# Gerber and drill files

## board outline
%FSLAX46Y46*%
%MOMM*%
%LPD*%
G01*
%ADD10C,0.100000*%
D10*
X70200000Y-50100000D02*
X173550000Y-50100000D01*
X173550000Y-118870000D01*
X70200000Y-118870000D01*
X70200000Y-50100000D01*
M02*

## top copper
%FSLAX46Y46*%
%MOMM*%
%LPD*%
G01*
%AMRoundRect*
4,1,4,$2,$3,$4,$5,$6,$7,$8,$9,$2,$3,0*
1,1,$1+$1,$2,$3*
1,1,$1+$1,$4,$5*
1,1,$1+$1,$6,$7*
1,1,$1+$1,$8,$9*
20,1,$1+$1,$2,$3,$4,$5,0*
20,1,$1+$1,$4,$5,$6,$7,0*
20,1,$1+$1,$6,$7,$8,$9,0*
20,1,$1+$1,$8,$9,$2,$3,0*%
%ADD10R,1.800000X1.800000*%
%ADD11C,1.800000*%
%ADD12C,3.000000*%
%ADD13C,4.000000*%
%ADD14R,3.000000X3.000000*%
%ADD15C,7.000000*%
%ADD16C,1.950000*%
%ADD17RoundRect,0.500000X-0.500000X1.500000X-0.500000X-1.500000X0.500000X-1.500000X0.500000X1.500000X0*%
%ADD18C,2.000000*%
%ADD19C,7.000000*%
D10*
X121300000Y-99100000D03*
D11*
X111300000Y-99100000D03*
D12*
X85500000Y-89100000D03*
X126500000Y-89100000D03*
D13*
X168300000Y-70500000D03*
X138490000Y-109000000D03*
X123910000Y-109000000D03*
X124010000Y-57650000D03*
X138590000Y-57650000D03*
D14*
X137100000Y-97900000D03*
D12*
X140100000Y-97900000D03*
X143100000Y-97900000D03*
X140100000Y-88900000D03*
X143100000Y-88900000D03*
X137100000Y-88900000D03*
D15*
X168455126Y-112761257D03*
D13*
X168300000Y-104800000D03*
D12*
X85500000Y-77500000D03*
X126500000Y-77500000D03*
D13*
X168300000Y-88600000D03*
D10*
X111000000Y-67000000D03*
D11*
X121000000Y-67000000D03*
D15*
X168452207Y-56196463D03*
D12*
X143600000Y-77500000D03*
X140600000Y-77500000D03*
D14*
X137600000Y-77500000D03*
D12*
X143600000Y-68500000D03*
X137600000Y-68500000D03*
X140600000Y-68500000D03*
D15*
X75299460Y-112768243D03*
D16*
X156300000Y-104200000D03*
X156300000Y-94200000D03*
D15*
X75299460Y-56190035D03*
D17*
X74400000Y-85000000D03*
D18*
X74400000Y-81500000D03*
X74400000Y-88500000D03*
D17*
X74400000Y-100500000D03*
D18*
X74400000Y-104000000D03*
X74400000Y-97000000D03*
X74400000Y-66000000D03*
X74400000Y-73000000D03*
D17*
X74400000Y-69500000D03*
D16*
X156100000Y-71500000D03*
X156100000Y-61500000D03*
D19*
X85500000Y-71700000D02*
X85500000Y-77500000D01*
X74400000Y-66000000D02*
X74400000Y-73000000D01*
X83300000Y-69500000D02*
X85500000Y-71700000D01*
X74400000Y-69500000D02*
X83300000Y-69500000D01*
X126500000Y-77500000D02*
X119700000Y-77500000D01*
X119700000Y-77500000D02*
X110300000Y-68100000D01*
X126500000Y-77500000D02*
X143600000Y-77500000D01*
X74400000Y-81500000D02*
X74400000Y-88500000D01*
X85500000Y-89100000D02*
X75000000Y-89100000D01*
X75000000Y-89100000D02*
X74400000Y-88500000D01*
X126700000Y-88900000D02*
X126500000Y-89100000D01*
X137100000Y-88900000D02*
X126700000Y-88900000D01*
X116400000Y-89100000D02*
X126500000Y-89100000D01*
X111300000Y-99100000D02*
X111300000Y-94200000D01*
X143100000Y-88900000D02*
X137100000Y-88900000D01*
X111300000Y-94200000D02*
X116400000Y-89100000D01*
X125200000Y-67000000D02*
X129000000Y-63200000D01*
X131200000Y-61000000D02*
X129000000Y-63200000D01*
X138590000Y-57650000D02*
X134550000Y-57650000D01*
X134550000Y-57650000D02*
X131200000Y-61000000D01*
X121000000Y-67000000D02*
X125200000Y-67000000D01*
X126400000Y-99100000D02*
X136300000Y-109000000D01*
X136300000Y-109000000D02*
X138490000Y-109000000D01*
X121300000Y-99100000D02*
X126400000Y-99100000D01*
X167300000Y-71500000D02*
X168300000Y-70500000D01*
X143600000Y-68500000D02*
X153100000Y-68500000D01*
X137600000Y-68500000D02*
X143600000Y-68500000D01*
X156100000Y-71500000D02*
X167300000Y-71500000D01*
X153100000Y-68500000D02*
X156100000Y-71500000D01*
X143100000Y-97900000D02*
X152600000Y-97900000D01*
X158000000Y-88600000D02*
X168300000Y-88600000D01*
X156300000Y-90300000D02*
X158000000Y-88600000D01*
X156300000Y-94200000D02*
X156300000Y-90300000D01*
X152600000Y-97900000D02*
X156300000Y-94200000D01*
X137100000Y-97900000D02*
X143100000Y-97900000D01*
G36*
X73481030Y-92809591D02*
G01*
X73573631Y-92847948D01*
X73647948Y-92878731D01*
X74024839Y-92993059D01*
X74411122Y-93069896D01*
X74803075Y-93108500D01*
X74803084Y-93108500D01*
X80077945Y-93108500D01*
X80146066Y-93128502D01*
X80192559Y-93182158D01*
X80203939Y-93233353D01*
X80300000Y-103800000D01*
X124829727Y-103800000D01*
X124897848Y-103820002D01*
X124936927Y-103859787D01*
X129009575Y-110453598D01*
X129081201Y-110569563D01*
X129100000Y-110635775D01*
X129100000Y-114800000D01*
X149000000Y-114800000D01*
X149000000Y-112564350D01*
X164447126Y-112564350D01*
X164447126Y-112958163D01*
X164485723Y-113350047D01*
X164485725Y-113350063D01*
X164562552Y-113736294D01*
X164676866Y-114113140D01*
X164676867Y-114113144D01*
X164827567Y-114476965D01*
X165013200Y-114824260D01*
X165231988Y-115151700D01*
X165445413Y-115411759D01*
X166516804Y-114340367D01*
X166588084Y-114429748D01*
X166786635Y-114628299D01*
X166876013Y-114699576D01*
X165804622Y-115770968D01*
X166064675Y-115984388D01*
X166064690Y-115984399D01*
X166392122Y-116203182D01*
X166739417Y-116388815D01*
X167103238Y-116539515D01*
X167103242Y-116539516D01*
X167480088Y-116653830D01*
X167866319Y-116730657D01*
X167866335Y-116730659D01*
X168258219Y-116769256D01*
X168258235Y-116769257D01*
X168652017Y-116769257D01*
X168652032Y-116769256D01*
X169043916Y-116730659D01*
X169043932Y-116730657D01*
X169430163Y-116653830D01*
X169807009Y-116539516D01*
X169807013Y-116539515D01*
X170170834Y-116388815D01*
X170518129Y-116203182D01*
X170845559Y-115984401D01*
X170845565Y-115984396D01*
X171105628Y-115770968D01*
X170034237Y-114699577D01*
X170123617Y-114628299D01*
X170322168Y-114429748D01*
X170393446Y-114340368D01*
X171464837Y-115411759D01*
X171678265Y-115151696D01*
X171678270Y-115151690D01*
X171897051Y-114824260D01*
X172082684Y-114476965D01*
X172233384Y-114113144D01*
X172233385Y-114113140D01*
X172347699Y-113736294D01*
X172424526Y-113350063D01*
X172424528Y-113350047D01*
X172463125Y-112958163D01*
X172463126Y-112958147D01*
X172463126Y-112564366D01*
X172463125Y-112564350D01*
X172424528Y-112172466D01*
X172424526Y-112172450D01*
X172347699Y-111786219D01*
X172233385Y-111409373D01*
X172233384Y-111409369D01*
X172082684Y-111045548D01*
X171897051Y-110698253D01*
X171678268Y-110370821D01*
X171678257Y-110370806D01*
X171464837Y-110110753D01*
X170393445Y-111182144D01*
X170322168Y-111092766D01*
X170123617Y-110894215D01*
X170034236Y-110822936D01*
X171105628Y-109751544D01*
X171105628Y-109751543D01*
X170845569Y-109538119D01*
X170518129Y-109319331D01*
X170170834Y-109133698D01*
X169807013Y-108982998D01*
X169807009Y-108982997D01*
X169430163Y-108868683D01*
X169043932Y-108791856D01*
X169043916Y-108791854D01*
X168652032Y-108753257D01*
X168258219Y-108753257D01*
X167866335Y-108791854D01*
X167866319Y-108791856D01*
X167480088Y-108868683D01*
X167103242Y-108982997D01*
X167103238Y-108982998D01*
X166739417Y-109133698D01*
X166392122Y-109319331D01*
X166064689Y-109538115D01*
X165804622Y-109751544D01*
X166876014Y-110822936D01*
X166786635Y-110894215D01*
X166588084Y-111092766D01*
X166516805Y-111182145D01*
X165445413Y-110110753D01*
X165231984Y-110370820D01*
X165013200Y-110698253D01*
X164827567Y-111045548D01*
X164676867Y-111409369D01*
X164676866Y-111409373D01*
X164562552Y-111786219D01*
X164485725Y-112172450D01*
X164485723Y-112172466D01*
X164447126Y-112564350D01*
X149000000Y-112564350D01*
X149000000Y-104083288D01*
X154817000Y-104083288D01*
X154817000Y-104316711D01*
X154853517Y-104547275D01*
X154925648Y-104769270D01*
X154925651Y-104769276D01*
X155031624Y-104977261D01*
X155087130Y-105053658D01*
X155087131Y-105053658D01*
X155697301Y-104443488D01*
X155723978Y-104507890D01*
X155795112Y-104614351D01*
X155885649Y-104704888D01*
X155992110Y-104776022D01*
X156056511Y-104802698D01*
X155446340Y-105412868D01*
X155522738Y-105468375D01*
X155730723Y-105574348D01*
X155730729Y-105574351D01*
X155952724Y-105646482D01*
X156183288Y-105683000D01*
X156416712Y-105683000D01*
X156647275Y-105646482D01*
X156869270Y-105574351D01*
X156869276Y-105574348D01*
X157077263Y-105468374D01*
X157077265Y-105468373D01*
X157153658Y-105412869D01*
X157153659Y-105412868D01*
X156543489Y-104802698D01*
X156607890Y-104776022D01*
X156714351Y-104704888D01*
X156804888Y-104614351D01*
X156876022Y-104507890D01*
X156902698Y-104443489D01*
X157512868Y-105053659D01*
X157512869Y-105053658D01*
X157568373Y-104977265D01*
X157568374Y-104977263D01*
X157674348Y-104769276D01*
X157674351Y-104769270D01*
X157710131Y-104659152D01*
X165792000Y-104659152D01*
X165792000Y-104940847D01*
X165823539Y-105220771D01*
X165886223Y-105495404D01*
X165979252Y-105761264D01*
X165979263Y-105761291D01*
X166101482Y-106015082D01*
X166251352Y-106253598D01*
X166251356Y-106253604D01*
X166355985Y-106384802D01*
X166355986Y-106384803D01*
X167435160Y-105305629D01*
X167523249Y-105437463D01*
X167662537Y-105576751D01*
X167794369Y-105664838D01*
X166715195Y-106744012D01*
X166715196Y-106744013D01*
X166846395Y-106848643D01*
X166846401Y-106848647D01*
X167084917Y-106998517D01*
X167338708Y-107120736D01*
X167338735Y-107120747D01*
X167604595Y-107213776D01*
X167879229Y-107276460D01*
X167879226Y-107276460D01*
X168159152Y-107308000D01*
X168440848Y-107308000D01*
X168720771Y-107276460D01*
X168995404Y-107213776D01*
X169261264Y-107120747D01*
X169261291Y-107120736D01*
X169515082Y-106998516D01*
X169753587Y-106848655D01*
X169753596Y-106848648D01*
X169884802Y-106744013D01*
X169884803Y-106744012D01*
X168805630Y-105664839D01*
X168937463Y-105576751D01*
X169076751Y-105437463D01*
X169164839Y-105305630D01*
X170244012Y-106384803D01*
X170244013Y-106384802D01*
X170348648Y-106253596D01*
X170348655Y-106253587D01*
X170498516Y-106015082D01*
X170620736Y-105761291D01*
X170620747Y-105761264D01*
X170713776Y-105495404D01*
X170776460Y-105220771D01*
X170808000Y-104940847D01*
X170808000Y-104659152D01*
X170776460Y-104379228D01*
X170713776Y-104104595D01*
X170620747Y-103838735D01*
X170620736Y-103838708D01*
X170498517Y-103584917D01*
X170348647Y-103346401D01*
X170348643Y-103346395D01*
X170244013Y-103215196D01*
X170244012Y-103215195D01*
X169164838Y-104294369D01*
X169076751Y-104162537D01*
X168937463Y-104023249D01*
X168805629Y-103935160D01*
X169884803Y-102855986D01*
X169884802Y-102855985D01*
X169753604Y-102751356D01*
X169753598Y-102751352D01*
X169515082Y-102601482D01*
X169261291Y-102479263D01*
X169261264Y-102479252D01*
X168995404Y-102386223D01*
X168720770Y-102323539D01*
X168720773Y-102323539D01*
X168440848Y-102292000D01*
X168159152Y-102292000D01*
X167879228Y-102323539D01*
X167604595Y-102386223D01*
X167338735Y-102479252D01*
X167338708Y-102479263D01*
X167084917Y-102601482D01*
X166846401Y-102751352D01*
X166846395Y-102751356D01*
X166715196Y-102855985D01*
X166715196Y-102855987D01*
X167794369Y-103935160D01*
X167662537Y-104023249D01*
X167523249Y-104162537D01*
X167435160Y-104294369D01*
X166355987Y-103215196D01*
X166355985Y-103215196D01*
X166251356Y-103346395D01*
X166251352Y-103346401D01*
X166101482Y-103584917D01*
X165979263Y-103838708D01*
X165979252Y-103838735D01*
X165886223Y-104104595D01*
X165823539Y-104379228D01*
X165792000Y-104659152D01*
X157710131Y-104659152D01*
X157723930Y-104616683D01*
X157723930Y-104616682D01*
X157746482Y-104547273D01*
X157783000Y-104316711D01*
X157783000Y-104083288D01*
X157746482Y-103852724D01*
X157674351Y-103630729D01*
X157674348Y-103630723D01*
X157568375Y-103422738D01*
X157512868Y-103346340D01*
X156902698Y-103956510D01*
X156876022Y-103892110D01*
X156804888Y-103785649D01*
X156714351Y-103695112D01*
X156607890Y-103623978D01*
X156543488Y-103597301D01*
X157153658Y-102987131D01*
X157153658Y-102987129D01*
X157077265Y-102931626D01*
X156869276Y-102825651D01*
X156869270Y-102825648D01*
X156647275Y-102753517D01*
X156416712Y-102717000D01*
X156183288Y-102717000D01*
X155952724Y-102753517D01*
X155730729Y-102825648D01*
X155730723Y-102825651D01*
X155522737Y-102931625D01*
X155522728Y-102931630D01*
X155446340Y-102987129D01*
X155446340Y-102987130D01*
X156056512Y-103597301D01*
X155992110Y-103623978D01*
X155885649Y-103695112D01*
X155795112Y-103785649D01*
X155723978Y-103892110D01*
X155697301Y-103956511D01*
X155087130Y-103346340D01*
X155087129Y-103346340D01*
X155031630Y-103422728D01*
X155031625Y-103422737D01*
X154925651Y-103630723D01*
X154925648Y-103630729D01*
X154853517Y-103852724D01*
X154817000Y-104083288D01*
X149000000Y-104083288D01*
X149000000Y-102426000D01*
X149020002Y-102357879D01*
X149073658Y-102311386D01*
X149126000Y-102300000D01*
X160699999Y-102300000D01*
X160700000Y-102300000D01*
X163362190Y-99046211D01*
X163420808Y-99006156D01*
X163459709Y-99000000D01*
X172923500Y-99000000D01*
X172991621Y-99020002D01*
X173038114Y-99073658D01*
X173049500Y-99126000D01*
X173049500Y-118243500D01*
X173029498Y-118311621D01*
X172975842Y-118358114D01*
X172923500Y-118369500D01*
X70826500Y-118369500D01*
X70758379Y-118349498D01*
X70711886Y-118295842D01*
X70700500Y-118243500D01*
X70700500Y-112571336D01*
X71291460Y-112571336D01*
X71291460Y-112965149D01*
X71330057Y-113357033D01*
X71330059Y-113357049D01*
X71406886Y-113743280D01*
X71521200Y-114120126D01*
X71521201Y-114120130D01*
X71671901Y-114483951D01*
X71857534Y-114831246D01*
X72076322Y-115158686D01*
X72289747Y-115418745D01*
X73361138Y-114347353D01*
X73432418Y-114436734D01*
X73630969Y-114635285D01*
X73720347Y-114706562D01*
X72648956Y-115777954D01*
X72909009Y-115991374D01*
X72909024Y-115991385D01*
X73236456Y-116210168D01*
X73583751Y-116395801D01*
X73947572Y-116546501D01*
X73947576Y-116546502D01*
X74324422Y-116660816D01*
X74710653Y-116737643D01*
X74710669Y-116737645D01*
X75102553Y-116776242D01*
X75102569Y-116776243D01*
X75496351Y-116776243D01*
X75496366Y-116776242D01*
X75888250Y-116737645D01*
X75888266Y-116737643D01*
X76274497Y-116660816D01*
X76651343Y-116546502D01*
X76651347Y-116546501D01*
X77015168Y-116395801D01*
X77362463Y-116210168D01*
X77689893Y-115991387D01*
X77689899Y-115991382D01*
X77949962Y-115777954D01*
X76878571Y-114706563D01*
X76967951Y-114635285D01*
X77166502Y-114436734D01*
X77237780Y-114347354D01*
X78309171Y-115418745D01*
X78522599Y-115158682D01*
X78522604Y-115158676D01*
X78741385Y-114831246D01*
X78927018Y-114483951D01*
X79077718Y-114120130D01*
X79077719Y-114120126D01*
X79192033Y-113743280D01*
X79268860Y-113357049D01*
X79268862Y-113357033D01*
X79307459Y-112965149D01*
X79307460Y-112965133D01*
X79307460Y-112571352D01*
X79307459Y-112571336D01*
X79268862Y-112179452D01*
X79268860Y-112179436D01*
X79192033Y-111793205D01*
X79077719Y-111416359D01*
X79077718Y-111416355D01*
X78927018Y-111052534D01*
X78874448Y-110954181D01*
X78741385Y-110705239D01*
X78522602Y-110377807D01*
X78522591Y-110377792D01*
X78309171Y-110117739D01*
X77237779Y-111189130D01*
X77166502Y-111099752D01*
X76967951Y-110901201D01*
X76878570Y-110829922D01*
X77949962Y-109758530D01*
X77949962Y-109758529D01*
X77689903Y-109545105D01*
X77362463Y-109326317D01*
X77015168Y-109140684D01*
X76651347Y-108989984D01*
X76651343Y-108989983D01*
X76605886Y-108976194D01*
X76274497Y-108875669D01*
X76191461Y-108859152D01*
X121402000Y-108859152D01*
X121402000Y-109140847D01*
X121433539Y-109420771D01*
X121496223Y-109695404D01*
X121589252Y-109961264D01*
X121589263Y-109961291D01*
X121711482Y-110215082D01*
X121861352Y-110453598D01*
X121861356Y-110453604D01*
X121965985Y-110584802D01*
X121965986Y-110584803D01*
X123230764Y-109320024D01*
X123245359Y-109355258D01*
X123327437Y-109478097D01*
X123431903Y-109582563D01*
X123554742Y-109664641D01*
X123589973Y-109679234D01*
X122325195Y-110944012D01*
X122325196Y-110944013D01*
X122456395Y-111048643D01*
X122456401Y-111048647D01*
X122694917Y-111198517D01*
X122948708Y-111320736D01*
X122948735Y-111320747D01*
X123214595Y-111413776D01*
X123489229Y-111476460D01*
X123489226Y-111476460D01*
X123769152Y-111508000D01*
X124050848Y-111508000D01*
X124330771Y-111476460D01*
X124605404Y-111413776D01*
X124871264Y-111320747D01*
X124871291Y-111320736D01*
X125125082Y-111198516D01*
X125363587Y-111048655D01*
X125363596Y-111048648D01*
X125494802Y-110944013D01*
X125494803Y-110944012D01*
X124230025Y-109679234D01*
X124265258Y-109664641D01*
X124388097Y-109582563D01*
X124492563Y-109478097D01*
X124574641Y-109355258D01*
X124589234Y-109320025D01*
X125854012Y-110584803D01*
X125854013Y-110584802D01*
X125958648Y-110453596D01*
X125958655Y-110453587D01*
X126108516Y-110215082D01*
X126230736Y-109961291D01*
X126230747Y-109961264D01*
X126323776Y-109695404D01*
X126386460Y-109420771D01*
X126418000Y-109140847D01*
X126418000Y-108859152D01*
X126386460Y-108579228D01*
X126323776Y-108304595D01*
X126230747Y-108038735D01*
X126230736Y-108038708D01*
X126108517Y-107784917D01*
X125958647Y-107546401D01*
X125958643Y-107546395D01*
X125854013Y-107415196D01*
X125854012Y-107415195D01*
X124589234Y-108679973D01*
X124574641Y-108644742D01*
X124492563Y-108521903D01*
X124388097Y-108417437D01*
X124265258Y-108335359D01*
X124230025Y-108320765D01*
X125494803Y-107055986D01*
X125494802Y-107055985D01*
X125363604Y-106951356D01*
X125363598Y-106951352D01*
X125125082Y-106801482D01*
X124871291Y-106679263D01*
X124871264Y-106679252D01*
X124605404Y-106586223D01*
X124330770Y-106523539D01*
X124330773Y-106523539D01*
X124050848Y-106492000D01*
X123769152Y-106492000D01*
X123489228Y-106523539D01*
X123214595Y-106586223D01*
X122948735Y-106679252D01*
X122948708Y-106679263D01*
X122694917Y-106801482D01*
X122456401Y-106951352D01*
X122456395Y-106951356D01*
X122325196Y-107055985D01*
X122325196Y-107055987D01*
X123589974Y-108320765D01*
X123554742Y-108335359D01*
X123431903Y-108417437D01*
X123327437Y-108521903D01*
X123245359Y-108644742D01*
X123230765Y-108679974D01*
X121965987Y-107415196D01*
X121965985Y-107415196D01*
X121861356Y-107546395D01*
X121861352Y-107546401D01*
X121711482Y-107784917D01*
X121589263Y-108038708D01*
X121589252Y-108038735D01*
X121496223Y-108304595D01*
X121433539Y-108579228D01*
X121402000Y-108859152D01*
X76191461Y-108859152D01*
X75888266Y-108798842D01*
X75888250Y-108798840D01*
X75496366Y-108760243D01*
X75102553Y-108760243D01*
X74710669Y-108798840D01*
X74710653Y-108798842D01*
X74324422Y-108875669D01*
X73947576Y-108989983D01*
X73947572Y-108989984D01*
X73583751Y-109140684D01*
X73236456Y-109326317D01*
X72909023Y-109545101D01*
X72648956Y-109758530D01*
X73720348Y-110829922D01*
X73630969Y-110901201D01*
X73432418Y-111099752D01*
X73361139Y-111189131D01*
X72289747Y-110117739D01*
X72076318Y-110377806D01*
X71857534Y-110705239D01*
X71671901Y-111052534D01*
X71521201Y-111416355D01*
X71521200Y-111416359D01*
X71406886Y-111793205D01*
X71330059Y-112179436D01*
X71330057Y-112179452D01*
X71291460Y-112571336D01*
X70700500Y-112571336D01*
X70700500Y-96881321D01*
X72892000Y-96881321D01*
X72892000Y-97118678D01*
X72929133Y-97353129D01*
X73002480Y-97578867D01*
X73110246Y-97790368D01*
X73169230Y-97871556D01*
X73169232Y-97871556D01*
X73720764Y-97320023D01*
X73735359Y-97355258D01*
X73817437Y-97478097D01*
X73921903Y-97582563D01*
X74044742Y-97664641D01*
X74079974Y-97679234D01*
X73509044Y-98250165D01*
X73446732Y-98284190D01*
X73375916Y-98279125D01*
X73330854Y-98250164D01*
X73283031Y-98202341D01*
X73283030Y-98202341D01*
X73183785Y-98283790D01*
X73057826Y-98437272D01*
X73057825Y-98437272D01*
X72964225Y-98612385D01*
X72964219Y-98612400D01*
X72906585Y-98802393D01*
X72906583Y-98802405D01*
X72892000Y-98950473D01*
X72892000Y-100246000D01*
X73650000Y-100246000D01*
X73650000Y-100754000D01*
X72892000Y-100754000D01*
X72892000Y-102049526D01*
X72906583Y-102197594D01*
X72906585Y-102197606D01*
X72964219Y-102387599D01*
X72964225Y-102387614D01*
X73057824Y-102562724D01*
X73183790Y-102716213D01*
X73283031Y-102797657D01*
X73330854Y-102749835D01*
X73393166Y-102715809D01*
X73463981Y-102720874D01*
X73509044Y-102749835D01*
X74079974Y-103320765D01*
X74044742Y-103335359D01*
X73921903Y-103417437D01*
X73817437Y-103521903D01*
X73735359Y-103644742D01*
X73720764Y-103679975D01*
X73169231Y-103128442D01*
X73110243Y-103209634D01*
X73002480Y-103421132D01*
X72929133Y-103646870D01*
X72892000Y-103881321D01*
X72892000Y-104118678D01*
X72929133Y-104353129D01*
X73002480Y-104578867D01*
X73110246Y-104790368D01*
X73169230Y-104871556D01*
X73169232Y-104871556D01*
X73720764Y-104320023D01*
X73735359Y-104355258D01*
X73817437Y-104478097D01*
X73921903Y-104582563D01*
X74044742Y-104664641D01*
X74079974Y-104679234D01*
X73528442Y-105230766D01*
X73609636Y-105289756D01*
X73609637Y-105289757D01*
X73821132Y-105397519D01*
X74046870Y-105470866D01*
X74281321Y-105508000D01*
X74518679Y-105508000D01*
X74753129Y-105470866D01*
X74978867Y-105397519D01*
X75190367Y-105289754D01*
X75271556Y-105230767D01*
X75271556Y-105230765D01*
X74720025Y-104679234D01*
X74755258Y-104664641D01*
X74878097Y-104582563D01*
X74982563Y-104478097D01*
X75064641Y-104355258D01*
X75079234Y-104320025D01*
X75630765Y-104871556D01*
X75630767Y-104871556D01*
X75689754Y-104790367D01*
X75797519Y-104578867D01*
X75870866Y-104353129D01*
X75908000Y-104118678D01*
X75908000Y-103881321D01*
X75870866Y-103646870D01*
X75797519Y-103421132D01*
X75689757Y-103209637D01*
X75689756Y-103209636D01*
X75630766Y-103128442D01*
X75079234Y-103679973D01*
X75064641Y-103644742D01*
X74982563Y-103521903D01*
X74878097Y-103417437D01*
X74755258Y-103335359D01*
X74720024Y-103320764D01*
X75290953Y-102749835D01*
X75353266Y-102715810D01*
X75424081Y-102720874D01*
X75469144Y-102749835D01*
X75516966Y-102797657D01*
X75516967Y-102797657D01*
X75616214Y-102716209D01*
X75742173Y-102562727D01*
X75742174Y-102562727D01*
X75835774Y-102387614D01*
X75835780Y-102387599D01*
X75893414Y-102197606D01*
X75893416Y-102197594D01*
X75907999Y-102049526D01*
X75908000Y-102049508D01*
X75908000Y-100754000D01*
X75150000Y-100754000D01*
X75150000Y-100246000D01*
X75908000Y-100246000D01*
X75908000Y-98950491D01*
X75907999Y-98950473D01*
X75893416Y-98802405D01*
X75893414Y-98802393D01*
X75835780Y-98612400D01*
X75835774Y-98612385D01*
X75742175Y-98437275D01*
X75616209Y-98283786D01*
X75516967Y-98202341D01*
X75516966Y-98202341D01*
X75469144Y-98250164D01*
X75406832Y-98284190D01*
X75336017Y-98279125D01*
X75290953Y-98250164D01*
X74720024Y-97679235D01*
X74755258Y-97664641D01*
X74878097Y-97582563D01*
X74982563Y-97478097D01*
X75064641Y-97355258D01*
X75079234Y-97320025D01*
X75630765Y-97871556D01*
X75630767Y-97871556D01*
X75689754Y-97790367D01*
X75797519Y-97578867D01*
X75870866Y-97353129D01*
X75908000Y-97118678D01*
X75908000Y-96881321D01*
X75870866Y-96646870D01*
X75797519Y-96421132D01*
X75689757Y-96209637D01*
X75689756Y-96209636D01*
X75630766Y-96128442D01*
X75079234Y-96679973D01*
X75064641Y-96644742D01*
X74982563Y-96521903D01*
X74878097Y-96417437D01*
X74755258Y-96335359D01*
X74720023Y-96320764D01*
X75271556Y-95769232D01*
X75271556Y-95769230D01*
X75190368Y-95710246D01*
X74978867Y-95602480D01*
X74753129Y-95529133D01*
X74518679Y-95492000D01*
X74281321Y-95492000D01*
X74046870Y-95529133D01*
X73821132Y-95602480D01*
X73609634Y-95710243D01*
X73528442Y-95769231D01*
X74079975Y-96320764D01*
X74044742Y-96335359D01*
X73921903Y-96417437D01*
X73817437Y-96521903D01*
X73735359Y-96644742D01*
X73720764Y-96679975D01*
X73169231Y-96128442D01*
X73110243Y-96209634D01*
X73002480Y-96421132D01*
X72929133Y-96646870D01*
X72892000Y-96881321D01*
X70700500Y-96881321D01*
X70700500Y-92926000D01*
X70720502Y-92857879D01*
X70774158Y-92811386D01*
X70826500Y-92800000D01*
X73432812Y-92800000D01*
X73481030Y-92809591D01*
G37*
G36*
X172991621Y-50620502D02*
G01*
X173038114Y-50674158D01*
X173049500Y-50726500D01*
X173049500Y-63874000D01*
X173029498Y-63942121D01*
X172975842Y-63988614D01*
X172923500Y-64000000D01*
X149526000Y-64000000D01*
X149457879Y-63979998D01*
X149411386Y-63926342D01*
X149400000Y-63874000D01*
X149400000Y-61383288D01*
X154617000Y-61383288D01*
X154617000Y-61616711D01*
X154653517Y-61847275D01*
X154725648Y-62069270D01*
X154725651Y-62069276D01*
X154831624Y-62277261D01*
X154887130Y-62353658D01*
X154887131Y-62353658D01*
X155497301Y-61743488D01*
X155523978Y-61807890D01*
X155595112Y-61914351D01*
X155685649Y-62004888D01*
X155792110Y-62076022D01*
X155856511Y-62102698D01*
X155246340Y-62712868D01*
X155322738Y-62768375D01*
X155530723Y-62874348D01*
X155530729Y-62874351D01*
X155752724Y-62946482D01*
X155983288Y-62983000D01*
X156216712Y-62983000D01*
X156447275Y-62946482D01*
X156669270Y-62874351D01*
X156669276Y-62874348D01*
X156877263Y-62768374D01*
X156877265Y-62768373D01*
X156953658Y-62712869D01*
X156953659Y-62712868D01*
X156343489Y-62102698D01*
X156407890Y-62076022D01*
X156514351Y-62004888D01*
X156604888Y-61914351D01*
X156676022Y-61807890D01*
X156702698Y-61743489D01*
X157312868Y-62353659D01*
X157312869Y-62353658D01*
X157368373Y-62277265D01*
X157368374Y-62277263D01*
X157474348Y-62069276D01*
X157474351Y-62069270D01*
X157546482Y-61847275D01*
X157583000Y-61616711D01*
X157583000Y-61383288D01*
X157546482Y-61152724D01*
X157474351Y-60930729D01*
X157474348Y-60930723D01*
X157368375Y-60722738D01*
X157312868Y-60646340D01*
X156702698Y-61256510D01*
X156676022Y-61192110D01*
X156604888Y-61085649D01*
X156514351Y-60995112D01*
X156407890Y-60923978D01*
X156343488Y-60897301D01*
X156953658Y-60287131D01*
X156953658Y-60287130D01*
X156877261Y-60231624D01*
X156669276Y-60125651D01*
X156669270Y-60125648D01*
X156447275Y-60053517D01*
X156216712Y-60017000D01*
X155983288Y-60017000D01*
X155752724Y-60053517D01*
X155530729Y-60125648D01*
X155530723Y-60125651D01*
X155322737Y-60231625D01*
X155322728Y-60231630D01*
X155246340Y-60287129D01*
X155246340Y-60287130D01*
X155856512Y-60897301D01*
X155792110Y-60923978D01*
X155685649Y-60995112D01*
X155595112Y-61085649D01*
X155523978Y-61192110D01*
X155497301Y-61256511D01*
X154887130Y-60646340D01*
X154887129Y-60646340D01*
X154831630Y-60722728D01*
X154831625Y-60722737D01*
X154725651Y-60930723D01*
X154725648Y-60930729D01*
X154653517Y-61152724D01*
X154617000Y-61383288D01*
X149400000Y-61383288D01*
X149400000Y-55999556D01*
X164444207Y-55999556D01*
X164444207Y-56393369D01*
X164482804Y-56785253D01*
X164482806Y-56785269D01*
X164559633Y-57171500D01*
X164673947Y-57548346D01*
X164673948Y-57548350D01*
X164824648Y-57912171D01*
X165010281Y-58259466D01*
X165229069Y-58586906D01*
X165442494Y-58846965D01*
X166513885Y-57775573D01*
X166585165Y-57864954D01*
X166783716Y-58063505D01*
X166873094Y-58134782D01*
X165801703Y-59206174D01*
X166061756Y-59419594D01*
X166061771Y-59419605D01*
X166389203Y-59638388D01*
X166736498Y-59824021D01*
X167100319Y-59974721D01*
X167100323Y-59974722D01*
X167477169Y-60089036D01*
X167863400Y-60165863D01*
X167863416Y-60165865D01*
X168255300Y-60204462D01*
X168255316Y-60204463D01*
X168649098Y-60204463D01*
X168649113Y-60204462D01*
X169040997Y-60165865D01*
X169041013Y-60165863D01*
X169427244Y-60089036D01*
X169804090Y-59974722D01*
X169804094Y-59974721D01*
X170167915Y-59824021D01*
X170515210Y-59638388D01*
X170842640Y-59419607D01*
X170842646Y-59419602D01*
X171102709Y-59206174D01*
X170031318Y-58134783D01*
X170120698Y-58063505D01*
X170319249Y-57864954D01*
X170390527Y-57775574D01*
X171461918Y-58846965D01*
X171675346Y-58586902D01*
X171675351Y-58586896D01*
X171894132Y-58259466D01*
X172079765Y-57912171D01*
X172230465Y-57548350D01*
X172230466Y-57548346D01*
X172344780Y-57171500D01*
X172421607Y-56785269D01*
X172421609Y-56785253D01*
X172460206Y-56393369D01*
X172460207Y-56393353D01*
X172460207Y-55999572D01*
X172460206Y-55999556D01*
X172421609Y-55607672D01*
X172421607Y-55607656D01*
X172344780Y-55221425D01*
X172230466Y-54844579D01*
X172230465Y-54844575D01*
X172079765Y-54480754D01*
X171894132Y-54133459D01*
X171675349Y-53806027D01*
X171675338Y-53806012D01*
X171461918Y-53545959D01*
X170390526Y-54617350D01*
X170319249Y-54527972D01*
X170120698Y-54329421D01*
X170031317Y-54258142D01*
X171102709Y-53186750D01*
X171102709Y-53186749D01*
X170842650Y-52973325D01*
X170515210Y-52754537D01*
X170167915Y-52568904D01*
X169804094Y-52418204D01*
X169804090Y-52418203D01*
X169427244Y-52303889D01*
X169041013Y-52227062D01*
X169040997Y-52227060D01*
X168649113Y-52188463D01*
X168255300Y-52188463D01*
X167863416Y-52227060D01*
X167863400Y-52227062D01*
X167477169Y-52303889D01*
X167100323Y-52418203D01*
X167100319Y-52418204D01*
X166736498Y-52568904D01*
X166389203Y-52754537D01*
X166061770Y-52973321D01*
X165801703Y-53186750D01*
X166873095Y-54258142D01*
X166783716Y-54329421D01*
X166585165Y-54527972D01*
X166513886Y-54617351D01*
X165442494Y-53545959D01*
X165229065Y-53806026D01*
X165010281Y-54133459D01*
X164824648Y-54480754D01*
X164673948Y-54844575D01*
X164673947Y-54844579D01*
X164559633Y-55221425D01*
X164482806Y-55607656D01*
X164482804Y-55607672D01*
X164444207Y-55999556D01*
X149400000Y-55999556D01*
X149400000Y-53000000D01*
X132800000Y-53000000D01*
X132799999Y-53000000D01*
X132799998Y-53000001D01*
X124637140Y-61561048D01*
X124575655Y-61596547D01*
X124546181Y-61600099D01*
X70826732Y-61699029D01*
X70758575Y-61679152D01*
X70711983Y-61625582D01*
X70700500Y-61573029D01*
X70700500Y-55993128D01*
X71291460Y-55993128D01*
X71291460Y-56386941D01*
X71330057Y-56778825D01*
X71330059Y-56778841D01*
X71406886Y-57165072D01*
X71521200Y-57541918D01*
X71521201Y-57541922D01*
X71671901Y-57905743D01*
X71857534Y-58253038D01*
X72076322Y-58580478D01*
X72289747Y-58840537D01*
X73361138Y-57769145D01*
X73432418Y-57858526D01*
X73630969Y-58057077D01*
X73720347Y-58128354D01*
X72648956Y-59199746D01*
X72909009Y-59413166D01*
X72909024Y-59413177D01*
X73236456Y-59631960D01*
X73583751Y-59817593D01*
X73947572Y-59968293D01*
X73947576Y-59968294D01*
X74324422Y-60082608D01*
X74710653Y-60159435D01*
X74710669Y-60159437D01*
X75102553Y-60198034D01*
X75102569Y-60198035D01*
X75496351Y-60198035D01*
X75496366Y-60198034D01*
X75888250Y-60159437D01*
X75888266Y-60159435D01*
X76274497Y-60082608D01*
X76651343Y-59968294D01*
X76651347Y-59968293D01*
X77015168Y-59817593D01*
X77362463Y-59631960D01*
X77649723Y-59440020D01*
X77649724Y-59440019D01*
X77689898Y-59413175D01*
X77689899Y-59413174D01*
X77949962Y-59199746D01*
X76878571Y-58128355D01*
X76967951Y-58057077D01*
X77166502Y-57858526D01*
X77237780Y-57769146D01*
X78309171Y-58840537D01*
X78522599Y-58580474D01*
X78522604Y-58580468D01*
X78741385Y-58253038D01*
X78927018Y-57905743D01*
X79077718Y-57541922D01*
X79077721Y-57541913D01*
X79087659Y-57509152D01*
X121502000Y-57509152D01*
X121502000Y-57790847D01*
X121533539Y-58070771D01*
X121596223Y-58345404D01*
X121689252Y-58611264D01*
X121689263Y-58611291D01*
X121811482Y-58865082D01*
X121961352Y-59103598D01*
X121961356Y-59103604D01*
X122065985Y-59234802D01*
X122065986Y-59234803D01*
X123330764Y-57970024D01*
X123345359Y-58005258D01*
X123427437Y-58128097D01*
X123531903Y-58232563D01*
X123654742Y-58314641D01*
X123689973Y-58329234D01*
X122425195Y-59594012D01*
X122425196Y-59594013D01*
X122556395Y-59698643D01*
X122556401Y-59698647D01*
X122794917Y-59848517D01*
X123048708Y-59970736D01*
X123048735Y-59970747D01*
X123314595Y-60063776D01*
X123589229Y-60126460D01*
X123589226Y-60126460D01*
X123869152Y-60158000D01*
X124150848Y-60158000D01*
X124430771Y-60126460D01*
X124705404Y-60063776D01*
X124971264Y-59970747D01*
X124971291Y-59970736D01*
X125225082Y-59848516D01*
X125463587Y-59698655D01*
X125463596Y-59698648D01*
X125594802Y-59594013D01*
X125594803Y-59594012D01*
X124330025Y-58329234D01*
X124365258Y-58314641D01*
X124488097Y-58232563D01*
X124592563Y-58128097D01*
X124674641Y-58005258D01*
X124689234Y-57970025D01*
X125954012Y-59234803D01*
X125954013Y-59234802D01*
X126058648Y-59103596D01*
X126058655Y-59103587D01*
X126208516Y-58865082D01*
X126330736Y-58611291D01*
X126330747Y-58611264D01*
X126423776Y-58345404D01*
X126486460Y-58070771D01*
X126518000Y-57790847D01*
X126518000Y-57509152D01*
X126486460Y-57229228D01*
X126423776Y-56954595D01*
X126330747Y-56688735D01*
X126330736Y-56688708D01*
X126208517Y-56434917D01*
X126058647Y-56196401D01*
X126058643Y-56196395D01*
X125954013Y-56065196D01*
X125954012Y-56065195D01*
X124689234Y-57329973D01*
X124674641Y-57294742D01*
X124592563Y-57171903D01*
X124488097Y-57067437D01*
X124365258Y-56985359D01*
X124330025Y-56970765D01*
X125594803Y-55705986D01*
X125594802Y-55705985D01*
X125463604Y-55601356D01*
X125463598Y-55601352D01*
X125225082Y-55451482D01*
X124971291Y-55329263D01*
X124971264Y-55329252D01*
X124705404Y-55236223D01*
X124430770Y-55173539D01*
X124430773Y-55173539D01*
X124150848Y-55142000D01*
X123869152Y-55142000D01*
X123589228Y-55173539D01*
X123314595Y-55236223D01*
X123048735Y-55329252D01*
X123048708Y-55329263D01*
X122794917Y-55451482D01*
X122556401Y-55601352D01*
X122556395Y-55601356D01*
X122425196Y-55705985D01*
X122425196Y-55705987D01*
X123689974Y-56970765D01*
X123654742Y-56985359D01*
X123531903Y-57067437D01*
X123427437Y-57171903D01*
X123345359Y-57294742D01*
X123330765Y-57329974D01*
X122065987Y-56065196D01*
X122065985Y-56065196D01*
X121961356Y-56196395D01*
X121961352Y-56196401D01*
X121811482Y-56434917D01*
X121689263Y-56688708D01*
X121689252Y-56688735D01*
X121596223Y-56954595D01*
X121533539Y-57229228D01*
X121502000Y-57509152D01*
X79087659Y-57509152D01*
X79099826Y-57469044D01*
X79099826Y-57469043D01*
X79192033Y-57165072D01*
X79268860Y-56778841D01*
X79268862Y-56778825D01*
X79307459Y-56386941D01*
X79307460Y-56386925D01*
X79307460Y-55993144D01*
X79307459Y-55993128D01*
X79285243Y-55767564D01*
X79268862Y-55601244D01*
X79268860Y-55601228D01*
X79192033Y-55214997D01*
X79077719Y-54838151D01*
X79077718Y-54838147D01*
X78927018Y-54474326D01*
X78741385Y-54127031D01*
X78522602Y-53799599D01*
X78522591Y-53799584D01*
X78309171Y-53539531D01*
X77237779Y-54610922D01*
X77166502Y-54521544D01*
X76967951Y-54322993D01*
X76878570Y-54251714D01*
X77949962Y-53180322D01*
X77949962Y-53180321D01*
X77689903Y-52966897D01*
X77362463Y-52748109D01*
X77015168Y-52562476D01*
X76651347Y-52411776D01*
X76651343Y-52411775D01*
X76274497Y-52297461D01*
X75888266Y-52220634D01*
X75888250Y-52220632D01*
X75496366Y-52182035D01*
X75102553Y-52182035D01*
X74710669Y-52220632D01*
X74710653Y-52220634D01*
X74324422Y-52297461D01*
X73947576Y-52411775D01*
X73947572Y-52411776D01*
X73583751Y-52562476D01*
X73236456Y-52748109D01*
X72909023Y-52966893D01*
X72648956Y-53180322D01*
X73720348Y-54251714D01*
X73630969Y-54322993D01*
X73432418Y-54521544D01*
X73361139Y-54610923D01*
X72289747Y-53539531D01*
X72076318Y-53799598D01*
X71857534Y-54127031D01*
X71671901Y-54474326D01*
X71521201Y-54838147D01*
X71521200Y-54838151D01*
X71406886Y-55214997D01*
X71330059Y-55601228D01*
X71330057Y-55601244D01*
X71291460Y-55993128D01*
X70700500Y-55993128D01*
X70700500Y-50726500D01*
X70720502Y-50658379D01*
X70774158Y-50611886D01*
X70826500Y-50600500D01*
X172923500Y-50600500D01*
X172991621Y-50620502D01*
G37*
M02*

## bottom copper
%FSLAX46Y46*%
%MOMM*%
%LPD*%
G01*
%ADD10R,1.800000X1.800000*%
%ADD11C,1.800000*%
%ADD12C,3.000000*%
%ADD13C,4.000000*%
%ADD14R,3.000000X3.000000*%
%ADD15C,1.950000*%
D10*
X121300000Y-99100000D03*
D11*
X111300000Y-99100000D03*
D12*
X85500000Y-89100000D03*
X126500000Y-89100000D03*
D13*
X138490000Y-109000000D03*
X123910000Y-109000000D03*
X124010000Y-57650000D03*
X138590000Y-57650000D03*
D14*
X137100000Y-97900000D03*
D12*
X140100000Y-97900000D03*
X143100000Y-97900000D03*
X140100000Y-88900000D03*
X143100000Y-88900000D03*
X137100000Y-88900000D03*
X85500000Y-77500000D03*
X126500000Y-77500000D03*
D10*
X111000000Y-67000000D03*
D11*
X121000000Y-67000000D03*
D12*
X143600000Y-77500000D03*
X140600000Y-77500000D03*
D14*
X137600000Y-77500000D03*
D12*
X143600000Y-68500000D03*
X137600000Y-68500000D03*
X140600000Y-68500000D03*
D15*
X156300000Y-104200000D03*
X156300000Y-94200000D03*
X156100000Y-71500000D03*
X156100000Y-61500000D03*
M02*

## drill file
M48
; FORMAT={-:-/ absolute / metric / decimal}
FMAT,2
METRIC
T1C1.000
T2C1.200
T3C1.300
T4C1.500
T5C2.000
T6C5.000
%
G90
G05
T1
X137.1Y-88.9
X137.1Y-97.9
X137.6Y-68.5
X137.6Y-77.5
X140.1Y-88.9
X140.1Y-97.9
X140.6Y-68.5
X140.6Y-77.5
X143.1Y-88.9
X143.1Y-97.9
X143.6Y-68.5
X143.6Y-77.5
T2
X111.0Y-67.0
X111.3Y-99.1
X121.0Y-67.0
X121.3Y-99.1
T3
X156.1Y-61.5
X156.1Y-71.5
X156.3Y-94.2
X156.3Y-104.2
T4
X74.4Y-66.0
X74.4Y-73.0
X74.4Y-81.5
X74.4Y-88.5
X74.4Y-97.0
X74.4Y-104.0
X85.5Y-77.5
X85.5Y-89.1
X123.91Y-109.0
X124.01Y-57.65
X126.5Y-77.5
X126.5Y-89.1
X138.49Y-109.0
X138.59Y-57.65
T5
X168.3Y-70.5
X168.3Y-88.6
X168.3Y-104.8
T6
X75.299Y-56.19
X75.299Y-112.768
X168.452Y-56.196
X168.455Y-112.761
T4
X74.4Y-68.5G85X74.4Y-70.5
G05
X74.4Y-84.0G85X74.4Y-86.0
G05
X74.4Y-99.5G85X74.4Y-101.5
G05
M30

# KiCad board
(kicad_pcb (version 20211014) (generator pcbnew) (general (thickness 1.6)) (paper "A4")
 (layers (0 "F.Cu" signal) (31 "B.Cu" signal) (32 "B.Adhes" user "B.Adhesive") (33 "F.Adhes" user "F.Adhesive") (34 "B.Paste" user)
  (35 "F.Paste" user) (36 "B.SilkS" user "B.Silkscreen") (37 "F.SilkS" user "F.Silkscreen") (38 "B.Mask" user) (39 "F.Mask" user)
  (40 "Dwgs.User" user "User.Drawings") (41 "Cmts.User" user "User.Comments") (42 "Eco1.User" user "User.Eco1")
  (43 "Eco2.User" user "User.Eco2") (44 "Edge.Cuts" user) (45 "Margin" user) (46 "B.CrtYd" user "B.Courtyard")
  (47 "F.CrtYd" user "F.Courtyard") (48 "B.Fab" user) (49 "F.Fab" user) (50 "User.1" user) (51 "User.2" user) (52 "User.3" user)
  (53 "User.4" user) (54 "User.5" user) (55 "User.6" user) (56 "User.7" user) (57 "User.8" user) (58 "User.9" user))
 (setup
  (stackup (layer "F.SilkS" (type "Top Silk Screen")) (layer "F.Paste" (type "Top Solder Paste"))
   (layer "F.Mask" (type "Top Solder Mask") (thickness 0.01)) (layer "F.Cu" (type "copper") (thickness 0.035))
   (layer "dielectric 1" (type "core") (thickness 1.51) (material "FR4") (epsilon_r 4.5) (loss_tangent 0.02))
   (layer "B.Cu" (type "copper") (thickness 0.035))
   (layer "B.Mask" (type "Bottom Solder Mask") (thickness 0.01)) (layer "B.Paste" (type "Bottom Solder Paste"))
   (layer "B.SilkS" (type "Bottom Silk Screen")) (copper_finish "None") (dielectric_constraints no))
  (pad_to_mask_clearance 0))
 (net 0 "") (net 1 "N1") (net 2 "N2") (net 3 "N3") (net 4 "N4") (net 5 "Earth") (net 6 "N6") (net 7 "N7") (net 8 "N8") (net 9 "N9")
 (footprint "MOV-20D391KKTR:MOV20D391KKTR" (layer "F.Cu") (at 121.3 99.1 180)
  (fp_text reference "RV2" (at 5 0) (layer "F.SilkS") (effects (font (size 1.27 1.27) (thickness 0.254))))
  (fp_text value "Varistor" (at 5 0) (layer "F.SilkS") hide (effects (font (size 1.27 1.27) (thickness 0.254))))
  (pad "1" thru_hole rect locked (at 0 0 180) (size 1.8 1.8) (drill 1.2) (layers *.Cu *.Mask) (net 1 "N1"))
  (pad "2" thru_hole circle locked (at 10 0 180) (size 1.8 1.8) (drill 1.2) (layers *.Cu *.Mask) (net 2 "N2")))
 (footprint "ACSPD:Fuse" (layer "F.Cu") (at 106 89.1)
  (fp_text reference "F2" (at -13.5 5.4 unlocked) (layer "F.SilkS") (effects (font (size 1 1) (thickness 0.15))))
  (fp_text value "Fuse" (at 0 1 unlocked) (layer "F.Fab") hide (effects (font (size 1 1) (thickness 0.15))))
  (pad "1" thru_hole circle (at -20.5 0) (size 3 3) (drill 1.5) (layers *.Cu *.Mask) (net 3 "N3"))
  (pad "2" thru_hole circle (at 20.5 0) (size 3 3) (drill 1.5) (layers *.Cu *.Mask) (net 2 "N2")))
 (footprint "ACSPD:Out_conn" (layer "F.Cu") (at 168.3 70.5)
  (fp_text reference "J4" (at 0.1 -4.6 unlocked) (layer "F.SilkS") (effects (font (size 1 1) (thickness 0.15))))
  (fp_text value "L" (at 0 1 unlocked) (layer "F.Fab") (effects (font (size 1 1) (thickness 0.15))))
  (pad "1" thru_hole circle (at 0 0) (size 4 4) (drill 2) (layers *.Cu *.Mask) (remove_unused_layers) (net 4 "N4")))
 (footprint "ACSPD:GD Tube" (layer "F.Cu") (at 131.2 109 180)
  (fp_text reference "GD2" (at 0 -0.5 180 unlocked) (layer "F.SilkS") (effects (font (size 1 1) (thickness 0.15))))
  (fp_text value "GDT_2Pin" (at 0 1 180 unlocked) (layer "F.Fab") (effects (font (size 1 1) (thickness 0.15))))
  (pad "1" thru_hole circle (at -7.29 0 180) (size 4 4) (drill 1.5) (layers *.Cu *.Mask) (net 1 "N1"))
  (pad "3" thru_hole circle (at 7.29 0 180) (size 4 4) (drill 1.5) (layers *.Cu *.Mask) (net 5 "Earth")))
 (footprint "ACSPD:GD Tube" (layer "F.Cu") (at 131.3 57.65)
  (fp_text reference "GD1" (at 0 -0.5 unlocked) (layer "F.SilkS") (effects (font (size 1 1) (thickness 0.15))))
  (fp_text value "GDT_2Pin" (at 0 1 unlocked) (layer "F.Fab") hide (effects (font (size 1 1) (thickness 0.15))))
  (pad "1" thru_hole circle (at -7.29 0) (size 4 4) (drill 1.5) (layers *.Cu *.Mask) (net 5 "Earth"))
  (pad "3" thru_hole circle (at 7.29 0) (size 4 4) (drill 1.5) (layers *.Cu *.Mask) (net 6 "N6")))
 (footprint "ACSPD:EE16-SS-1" (layer "F.Cu") (at 140.1 93.4 180)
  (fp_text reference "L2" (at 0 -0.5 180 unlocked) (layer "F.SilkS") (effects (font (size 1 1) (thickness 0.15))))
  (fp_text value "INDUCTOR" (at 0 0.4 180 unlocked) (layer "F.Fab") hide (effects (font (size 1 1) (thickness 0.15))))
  (pad "1" thru_hole rect (at 3 -4.5 180) (size 3 3) (drill 1) (layers *.Cu *.Mask) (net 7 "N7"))
  (pad "1" thru_hole circle (at 0 -4.5 180) (size 3 3) (drill 1) (layers *.Cu *.Mask) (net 7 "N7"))
  (pad "1" thru_hole circle (at -3 -4.5 180) (size 3 3) (drill 1) (layers *.Cu *.Mask) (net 7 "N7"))
  (pad "2" thru_hole circle (at 0 4.5 180) (size 3 3) (drill 1) (layers *.Cu *.Mask) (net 2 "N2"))
  (pad "2" thru_hole circle (at -3 4.5 180) (size 3 3) (drill 1) (layers *.Cu *.Mask) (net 2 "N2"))
  (pad "2" thru_hole circle (at 3 4.5 180) (size 3 3) (drill 1) (layers *.Cu *.Mask) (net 2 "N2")))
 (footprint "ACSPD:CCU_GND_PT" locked (layer "F.Cu") (at 168.455126 112.761257)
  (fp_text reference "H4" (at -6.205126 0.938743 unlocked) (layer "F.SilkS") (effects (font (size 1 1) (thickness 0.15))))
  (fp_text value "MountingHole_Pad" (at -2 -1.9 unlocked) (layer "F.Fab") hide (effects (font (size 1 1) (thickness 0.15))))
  (pad "1" thru_hole circle locked (at 0 0) (size 7 7) (drill 5) (layers *.Cu *.Mask) (remove_unused_layers) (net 5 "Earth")))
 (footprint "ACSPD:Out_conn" (layer "F.Cu") (at 168.3 104.8)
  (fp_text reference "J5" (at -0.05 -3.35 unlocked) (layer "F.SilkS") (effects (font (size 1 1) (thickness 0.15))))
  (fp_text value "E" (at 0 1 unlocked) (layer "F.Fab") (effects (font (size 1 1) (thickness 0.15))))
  (pad "1" thru_hole circle (at 0 0) (size 4 4) (drill 2) (layers *.Cu *.Mask) (remove_unused_layers) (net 5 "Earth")))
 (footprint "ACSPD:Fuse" (layer "F.Cu") (at 106 77.5)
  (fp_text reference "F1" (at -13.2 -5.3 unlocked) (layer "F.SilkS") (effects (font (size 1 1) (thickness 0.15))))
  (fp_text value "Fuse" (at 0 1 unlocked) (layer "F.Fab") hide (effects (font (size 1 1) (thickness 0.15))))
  (pad "1" thru_hole circle (at -20.5 0) (size 3 3) (drill 1.5) (layers *.Cu *.Mask) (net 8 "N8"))
  (pad "2" thru_hole circle (at 20.5 0) (size 3 3) (drill 1.5) (layers *.Cu *.Mask) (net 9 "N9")))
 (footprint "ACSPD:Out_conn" (layer "F.Cu") (at 168.3 88.6)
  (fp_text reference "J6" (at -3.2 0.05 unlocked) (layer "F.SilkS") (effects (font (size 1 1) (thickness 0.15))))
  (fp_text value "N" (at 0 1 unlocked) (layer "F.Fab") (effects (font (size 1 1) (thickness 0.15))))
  (pad "1" thru_hole circle (at 0 0) (size 4 4) (drill 2) (layers *.Cu *.Mask) (remove_unused_layers) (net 7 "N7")))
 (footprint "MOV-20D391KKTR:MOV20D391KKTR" (layer "F.Cu") (at 111 67)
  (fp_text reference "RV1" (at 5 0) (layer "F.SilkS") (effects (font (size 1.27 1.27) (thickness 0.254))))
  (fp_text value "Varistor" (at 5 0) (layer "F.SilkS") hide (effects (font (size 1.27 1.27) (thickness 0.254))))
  (pad "1" thru_hole rect locked (at 0 0) (size 1.8 1.8) (drill 1.2) (layers *.Cu *.Mask) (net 9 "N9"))
  (pad "2" thru_hole circle locked (at 10 0) (size 1.8 1.8) (drill 1.2) (layers *.Cu *.Mask) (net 6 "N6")))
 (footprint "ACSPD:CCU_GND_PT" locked (layer "F.Cu") (at 168.452207 56.196463)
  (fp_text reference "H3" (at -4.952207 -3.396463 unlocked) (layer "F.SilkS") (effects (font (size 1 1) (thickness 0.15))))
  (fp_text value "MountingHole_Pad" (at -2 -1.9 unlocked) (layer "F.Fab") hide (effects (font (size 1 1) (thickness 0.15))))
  (pad "1" thru_hole circle locked (at 0 0) (size 7 7) (drill 5) (layers *.Cu *.Mask) (remove_unused_layers) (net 5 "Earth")))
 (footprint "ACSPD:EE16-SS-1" (layer "F.Cu") (at 140.6 73 180)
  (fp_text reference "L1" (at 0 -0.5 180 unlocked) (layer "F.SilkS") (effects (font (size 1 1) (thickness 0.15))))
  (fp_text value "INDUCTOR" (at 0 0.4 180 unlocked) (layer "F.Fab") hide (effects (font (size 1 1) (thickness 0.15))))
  (pad "1" thru_hole circle (at -3 -4.5 180) (size 3 3) (drill 1) (layers *.Cu *.Mask) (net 9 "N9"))
  (pad "1" thru_hole circle (at 0 -4.5 180) (size 3 3) (drill 1) (layers *.Cu *.Mask) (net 9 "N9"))
  (pad "1" thru_hole rect (at 3 -4.5 180) (size 3 3) (drill 1) (layers *.Cu *.Mask) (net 9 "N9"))
  (pad "2" thru_hole circle (at -3 4.5 180) (size 3 3) (drill 1) (layers *.Cu *.Mask) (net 4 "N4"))
  (pad "2" thru_hole circle (at 3 4.5 180) (size 3 3) (drill 1) (layers *.Cu *.Mask) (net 4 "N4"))
  (pad "2" thru_hole circle (at 0 4.5 180) (size 3 3) (drill 1) (layers *.Cu *.Mask) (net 4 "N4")))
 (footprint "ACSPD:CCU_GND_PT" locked (layer "F.Cu") (at 75.29946 112.768243)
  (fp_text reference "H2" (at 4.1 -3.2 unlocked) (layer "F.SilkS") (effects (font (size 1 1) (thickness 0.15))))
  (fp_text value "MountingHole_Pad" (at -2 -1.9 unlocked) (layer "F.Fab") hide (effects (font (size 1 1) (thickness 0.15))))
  (pad "1" thru_hole circle locked (at 0 0) (size 7 7) (drill 5) (layers *.Cu *.Mask) (remove_unused_layers) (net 5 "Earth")))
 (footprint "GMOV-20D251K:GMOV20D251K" (layer "F.Cu") (at 156.3 104.2 90)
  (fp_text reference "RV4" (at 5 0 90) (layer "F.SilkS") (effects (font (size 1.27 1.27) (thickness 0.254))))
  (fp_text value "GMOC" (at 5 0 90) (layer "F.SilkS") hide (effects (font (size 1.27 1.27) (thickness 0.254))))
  (pad "1" thru_hole circle locked (at 0 0 90) (size 1.95 1.95) (drill 1.3) (layers *.Cu *.Mask) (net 5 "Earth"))
  (pad "2" thru_hole circle locked (at 10 0 90) (size 1.95 1.95) (drill 1.3) (layers *.Cu *.Mask) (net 7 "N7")))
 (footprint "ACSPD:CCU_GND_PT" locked (layer "F.Cu") (at 75.29946 56.190035)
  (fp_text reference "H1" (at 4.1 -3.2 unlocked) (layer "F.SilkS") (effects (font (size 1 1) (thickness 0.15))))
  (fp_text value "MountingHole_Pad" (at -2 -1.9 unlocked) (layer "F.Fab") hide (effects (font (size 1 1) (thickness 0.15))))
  (pad "1" thru_hole circle locked (at 0 0) (size 7 7) (drill 5) (layers *.Cu *.Mask) (remove_unused_layers) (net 5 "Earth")))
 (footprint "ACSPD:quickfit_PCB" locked (layer "F.Cu") (at 74.4 85 -90)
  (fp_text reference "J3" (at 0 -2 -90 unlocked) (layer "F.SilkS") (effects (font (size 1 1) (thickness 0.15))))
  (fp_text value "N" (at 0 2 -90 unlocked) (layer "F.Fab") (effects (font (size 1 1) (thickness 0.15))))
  (pad "1" thru_hole roundrect locked (at 0 0 270) (size 4 2) (drill oval 3.5 1.5) (layers *.Cu *.Mask) (remove_unused_layers)
   (roundrect_rratio 0.25) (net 3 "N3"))
  (pad "1" thru_hole circle locked (at -3.5 0 270) (size 2 2) (drill 1.5) (layers *.Cu *.Mask) (remove_unused_layers) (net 3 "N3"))
  (pad "1" thru_hole circle locked (at 3.5 0 270) (size 2 2) (drill 1.5) (layers *.Cu *.Mask) (remove_unused_layers) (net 3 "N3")))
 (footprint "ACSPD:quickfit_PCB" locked (layer "F.Cu") (at 74.4 100.5 -90)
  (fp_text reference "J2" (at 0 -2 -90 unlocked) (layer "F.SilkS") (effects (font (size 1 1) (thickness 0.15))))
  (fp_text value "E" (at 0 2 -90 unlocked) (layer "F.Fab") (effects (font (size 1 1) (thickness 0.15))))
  (pad "1" thru_hole roundrect locked (at 0 0 270) (size 4 2) (drill oval 3.5 1.5) (layers *.Cu *.Mask) (remove_unused_layers)
   (roundrect_rratio 0.25) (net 5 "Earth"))
  (pad "1" thru_hole circle locked (at 3.5 0 270) (size 2 2) (drill 1.5) (layers *.Cu *.Mask) (remove_unused_layers) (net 5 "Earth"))
  (pad "1" thru_hole circle locked (at -3.5 0 270) (size 2 2) (drill 1.5) (layers *.Cu *.Mask) (remove_unused_layers) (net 5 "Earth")))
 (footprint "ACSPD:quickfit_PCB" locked (layer "F.Cu") (at 74.4 69.5 -90)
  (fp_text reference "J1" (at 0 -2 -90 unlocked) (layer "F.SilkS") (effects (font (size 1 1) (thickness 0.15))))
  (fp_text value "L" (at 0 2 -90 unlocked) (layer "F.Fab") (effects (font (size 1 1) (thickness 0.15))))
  (pad "1" thru_hole circle locked (at -3.5 0 270) (size 2 2) (drill 1.5) (layers *.Cu *.Mask) (remove_unused_layers) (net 8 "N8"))
  (pad "1" thru_hole circle locked (at 3.5 0 270) (size 2 2) (drill 1.5) (layers *.Cu *.Mask) (remove_unused_layers) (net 8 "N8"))
  (pad "1" thru_hole roundrect locked (at 0 0 270) (size 4 2) (drill oval 3.5 1.5) (layers *.Cu *.Mask) (remove_unused_layers)
   (roundrect_rratio 0.25) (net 8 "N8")))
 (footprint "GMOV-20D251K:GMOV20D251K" (layer "F.Cu") (at 156.1 71.5 90)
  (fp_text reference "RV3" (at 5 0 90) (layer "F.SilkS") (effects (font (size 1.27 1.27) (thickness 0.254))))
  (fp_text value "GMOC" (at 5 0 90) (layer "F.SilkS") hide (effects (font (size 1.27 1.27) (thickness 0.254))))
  (pad "1" thru_hole circle locked (at 0 0 90) (size 1.95 1.95) (drill 1.3) (layers *.Cu *.Mask) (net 4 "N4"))
  (pad "2" thru_hole circle locked (at 10 0 90) (size 1.95 1.95) (drill 1.3) (layers *.Cu *.Mask) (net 5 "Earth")))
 (gr_rect (start 70.2 50.1) (end 173.55 118.87) (layer "Edge.Cuts") (width 0.1) (fill none))
 (segment (start 85.5 71.7) (end 85.5 77.5) (width 7) (layer "F.Cu") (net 8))
 (segment (start 74.4 66) (end 74.4 73) (width 7) (layer "F.Cu") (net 8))
 (segment (start 83.3 69.5) (end 85.5 71.7) (width 7) (layer "F.Cu") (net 8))
 (segment (start 74.4 69.5) (end 83.3 69.5) (width 7) (layer "F.Cu") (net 8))
 (segment (start 126.5 77.5) (end 119.7 77.5) (width 7) (layer "F.Cu") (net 9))
 (segment (start 119.7 77.5) (end 110.3 68.1) (width 7) (layer "F.Cu") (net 9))
 (segment (start 126.5 77.5) (end 143.6 77.5) (width 7) (layer "F.Cu") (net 9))
 (segment (start 74.4 81.5) (end 74.4 88.5) (width 7) (layer "F.Cu") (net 3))
 (segment (start 85.5 89.1) (end 75 89.1) (width 7) (layer "F.Cu") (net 3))
 (segment (start 75 89.1) (end 74.4 88.5) (width 7) (layer "F.Cu") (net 3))
 (segment (start 126.7 88.9) (end 126.5 89.1) (width 7) (layer "F.Cu") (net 2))
 (segment (start 137.1 88.9) (end 126.7 88.9) (width 7) (layer "F.Cu") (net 2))
 (segment (start 116.4 89.1) (end 126.5 89.1) (width 7) (layer "F.Cu") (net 2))
 (segment (start 111.3 99.1) (end 111.3 94.2) (width 7) (layer "F.Cu") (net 2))
 (segment (start 143.1 88.9) (end 137.1 88.9) (width 7) (layer "F.Cu") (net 2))
 (segment (start 111.3 94.2) (end 116.4 89.1) (width 7) (layer "F.Cu") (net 2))
 (segment (start 125.2 67) (end 129 63.2) (width 7) (layer "F.Cu") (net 6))
 (segment (start 131.2 61) (end 129 63.2) (width 7) (layer "F.Cu") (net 6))
 (segment (start 138.59 57.65) (end 134.55 57.65) (width 7) (layer "F.Cu") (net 6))
 (segment (start 134.55 57.65) (end 131.2 61) (width 7) (layer "F.Cu") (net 6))
 (segment (start 121 67) (end 125.2 67) (width 7) (layer "F.Cu") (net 6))
 (segment (start 126.4 99.1) (end 136.3 109) (width 7) (layer "F.Cu") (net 1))
 (segment (start 136.3 109) (end 138.49 109) (width 7) (layer "F.Cu") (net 1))
 (segment (start 121.3 99.1) (end 126.4 99.1) (width 7) (layer "F.Cu") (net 1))
 (segment (start 167.3 71.5) (end 168.3 70.5) (width 7) (layer "F.Cu") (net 4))
 (segment (start 143.6 68.5) (end 153.1 68.5) (width 7) (layer "F.Cu") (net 4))
 (segment (start 137.6 68.5) (end 143.6 68.5) (width 7) (layer "F.Cu") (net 4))
 (segment (start 156.1 71.5) (end 167.3 71.5) (width 7) (layer "F.Cu") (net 4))
 (segment (start 153.1 68.5) (end 156.1 71.5) (width 7) (layer "F.Cu") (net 4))
 (segment (start 143.1 97.9) (end 152.6 97.9) (width 7) (layer "F.Cu") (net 7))
 (segment (start 158 88.6) (end 168.3 88.6) (width 7) (layer "F.Cu") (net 7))
 (segment (start 156.3 90.3) (end 158 88.6) (width 7) (layer "F.Cu") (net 7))
 (segment (start 156.3 94.2) (end 156.3 90.3) (width 7) (layer "F.Cu") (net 7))
 (segment (start 152.6 97.9) (end 156.3 94.2) (width 7) (layer "F.Cu") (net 7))
 (segment (start 137.1 97.9) (end 143.1 97.9) (width 7) (layer "F.Cu") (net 7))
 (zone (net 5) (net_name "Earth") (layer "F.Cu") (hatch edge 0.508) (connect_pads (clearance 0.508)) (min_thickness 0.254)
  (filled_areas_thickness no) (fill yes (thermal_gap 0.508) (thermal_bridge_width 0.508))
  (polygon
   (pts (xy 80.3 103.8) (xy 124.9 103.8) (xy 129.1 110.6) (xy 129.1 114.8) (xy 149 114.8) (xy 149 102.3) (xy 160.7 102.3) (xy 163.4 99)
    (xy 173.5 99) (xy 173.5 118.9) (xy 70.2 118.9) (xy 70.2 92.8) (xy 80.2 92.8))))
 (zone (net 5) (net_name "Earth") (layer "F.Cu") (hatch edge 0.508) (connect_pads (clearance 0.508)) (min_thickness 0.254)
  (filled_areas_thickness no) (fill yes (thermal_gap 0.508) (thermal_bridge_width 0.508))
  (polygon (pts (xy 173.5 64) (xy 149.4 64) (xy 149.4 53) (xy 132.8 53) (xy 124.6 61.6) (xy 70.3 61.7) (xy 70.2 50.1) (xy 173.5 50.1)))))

